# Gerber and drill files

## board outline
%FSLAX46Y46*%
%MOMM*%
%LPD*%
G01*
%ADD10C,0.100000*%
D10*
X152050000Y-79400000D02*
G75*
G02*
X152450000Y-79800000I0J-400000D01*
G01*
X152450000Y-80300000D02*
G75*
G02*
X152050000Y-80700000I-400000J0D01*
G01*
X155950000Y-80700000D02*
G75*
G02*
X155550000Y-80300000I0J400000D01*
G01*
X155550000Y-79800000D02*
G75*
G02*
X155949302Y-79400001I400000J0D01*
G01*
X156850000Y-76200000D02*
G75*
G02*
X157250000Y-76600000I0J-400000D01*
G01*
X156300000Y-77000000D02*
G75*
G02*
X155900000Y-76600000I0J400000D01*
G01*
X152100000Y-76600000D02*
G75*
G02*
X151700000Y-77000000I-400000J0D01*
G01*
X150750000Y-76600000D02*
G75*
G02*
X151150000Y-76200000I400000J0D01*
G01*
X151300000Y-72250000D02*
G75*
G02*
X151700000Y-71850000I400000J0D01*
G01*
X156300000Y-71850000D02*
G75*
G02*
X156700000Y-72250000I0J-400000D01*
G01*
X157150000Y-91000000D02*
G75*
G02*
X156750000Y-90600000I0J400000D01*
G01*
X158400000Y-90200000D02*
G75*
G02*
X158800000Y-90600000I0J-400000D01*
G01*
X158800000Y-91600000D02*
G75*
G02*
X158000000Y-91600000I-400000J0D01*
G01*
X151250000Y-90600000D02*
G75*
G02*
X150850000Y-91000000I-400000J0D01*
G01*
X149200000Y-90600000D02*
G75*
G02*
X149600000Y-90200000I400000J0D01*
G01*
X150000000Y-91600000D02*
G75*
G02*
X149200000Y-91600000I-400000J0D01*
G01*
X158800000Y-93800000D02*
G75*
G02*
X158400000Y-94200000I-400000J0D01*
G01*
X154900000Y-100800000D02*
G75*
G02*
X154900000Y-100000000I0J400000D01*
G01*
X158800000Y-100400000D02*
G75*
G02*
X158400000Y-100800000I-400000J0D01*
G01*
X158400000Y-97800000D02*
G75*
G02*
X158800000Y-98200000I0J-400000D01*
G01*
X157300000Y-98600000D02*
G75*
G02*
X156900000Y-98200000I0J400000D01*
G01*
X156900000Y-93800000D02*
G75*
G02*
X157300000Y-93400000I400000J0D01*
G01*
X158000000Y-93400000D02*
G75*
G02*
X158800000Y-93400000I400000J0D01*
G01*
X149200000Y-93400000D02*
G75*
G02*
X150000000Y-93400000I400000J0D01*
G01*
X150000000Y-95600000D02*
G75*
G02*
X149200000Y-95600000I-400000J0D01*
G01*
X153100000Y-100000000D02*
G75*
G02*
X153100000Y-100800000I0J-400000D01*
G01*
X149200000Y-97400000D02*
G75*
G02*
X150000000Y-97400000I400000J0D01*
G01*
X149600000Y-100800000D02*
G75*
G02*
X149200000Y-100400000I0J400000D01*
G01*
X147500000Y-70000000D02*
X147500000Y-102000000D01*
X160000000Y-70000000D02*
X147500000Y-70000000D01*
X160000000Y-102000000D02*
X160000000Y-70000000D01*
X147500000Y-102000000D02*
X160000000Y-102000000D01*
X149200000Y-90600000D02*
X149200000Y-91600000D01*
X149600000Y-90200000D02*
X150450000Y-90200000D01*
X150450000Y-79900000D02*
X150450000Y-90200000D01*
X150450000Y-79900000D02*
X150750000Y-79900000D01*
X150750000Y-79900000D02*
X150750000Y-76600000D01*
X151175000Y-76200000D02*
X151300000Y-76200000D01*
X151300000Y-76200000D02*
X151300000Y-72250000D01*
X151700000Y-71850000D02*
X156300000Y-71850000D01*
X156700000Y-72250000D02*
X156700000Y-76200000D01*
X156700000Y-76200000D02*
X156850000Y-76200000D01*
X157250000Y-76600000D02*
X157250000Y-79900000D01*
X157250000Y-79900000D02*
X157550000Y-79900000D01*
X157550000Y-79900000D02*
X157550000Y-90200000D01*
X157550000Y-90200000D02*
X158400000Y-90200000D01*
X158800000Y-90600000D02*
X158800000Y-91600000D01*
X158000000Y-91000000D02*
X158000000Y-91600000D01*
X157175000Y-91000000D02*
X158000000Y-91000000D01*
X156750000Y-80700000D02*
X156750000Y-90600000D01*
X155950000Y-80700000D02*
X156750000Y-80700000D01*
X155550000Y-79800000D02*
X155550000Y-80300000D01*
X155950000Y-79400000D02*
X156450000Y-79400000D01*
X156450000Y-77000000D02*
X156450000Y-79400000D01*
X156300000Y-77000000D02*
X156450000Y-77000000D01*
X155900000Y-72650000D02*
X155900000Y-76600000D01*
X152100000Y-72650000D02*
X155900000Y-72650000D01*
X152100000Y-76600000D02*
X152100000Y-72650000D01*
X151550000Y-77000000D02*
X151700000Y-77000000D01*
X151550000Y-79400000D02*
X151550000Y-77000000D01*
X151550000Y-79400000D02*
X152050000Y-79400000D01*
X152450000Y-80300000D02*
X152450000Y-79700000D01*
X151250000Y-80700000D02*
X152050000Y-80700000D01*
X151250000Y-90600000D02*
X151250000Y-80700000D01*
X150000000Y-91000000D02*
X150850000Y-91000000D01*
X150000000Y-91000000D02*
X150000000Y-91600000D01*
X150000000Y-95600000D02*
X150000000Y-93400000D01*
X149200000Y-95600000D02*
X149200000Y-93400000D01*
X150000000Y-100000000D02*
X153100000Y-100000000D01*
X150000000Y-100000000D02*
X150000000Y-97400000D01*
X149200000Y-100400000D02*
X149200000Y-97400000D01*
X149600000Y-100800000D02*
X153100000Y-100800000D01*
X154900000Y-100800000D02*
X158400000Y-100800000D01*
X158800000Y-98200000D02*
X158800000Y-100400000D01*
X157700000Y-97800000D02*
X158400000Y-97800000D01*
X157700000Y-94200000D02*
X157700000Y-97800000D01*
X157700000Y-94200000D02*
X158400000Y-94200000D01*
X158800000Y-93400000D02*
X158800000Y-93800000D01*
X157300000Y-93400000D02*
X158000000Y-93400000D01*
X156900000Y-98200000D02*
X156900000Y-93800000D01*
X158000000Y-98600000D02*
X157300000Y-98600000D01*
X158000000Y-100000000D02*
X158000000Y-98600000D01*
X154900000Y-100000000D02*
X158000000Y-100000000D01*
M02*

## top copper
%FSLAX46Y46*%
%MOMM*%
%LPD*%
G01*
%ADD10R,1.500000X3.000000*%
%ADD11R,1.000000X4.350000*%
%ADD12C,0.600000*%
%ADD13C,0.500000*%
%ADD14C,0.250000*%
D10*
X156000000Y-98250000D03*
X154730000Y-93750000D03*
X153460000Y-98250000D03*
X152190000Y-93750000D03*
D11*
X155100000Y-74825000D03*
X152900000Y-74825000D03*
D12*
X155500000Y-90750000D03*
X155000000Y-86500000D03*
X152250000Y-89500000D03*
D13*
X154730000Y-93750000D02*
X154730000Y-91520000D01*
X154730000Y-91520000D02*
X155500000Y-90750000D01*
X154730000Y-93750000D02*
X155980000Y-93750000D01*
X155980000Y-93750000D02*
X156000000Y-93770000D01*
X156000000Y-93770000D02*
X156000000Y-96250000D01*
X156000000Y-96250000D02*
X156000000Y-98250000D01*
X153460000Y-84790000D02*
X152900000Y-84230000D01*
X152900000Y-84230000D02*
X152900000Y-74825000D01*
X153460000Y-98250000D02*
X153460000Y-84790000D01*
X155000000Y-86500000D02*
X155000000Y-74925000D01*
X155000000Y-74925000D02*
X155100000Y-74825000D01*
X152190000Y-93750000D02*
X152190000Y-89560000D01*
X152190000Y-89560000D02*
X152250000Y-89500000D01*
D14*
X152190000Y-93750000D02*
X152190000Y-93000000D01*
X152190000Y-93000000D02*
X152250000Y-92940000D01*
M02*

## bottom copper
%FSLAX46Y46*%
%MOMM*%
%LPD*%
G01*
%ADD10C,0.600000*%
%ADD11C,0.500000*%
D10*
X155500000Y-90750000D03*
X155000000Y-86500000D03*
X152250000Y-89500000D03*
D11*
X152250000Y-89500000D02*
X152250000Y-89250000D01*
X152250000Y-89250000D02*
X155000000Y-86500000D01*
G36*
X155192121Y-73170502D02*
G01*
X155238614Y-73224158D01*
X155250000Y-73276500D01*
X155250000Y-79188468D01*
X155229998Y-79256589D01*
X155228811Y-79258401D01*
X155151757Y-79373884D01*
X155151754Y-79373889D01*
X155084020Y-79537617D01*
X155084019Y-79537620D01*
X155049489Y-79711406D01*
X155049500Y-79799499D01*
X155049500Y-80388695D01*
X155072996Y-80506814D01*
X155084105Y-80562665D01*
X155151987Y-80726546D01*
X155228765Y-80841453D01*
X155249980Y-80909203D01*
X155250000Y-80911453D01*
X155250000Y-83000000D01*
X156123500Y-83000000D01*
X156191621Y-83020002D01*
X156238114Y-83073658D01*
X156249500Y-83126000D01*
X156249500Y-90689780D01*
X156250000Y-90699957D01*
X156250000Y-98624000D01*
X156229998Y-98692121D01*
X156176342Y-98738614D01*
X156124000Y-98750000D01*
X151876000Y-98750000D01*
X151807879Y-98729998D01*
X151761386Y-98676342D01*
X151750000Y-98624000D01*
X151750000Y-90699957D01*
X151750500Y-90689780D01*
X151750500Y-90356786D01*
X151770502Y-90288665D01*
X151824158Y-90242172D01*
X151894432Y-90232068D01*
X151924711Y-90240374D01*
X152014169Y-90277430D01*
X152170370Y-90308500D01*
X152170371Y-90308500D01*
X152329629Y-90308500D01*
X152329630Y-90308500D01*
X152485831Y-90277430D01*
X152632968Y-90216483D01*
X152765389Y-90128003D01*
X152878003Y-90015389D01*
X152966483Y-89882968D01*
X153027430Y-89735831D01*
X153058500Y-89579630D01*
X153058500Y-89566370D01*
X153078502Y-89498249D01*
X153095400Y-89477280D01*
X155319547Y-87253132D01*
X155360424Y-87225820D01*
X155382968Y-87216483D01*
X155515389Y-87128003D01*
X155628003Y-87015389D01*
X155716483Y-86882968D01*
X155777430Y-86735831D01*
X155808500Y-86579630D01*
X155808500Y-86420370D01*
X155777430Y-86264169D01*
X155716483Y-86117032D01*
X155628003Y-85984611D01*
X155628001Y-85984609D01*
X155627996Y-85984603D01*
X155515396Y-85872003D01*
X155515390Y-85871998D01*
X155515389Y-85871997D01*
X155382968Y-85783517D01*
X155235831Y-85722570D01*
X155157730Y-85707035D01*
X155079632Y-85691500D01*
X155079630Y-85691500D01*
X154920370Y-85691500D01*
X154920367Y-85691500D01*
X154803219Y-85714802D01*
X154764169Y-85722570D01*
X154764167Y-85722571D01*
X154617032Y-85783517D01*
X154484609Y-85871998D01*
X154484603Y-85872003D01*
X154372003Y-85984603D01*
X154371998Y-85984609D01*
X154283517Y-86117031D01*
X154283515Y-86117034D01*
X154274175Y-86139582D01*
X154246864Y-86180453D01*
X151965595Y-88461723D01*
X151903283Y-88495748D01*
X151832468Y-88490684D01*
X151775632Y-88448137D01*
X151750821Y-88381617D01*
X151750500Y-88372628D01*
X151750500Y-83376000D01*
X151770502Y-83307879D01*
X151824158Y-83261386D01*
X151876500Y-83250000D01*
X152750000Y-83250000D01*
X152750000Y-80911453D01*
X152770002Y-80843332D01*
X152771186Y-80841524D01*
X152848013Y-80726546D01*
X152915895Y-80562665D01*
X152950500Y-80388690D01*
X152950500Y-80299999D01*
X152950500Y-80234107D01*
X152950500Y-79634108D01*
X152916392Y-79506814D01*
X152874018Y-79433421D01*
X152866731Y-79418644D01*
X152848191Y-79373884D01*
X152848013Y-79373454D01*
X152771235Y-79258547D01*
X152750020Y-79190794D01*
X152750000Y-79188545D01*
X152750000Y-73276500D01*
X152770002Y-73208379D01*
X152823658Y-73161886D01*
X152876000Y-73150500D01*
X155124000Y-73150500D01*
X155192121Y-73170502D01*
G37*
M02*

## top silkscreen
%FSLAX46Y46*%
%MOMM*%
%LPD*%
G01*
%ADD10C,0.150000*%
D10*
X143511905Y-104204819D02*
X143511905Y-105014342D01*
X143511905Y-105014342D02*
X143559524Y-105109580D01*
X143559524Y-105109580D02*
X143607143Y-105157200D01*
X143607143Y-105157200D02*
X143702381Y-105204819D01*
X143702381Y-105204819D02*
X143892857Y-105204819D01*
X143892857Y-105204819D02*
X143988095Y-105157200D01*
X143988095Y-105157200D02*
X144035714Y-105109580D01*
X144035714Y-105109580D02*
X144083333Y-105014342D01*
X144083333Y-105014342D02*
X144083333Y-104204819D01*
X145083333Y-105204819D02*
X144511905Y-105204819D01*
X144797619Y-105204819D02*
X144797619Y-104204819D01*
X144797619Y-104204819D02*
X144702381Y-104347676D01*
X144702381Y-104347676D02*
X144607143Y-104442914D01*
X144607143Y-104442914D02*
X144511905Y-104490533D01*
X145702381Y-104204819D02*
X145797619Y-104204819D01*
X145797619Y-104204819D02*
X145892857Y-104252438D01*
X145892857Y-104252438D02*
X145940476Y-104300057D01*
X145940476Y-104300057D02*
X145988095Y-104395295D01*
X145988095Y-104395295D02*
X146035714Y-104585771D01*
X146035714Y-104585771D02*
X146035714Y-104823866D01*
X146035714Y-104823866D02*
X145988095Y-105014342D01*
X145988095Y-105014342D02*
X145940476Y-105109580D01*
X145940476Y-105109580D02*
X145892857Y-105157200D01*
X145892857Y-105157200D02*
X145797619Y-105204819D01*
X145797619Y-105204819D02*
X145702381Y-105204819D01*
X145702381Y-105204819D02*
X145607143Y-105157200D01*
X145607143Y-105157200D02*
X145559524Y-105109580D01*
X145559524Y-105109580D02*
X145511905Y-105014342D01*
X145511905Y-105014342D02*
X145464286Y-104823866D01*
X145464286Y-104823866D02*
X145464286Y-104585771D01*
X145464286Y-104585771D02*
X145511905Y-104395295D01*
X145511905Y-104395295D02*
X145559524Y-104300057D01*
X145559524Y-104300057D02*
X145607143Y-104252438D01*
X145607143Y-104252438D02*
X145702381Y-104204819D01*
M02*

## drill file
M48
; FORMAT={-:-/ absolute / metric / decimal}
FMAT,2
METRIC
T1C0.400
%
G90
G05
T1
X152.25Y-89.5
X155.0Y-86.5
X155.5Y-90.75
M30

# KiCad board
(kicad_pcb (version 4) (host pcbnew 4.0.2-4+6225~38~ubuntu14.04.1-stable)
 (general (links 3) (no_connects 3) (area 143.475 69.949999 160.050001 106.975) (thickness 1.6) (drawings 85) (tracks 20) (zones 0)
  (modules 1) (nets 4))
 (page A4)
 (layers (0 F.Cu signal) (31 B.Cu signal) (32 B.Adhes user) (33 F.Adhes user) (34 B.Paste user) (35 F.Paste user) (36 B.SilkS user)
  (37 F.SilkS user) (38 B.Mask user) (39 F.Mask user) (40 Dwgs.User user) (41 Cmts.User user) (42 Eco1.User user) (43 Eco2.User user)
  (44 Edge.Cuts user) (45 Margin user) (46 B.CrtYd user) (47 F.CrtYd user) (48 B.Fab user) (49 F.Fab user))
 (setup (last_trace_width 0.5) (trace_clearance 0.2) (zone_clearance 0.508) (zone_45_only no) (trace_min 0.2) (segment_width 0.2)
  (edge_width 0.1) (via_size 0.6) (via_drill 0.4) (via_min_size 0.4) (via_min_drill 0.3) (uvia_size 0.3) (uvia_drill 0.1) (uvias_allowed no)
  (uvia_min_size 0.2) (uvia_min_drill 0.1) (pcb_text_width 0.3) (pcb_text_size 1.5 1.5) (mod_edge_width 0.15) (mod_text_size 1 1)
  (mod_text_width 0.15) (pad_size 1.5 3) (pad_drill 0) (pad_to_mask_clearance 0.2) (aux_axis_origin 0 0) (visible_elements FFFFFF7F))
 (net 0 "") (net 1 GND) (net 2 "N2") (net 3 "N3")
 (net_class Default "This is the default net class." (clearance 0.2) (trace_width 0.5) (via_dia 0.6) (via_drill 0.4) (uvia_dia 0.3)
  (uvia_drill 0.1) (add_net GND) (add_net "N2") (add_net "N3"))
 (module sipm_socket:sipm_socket (layer F.Cu) (at 150 100)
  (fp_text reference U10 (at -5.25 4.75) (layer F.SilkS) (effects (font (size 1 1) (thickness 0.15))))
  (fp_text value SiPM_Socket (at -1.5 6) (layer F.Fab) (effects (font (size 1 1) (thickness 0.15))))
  (pad 1 smd rect (at 6 -1.75) (size 1.5 3) (layers F.Cu F.Paste F.Mask) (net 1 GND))
  (pad 2 smd rect (at 4.73 -6.25) (size 1.5 3) (layers F.Cu F.Paste F.Mask) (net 1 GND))
  (pad 3 smd rect (at 3.46 -1.75) (size 1.5 3) (layers F.Cu F.Paste F.Mask) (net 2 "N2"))
  (pad 4 smd rect (at 2.19 -6.25) (size 1.5 3) (layers F.Cu F.Paste F.Mask) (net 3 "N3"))
  (pad 5 smd rect (at 5.1 -25.175) (size 1 4.35) (layers F.Cu F.Paste F.Mask) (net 3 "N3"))
  (pad 6 smd rect (at 2.9 -25.175) (size 1 4.35) (layers F.Cu F.Paste F.Mask) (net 2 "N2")))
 (gr_arc (start 152.05 79.8) (end 152.05 79.4) (angle 90) (layer Edge.Cuts) (width 0.1))
 (gr_arc (start 152.05 80.3) (end 152.45 80.3) (angle 90) (layer Edge.Cuts) (width 0.1))
 (gr_arc (start 155.95 80.3) (end 155.55 80.3) (angle -90) (layer Edge.Cuts) (width 0.1))
 (gr_arc (start 155.95 79.8) (end 155.55 79.8) (angle 89.9) (layer Edge.Cuts) (width 0.1))
 (gr_arc (start 156.85 76.6) (end 157.25 76.6) (angle -90) (layer Edge.Cuts) (width 0.1))
 (gr_arc (start 156.3 76.6) (end 156.3 77) (angle 90) (layer Edge.Cuts) (width 0.1))
 (gr_arc (start 151.7 76.6) (end 152.1 76.6) (angle 90) (layer Edge.Cuts) (width 0.1))
 (gr_arc (start 151.15 76.6) (end 150.75 76.6) (angle 90) (layer Edge.Cuts) (width 0.1))
 (gr_arc (start 151.7 72.25) (end 151.3 72.25) (angle 90) (layer Edge.Cuts) (width 0.1))
 (gr_arc (start 156.3 72.25) (end 156.7 72.25) (angle -90) (layer Edge.Cuts) (width 0.1))
 (gr_arc (start 157.15 90.6) (end 156.75 90.6) (angle -90) (layer Edge.Cuts) (width 0.1))
 (gr_arc (start 158.4 90.6) (end 158.4 90.2) (angle 90) (layer Edge.Cuts) (width 0.1))
 (gr_arc (start 158.4 91.6) (end 158 91.6) (angle -180) (layer Edge.Cuts) (width 0.1))
 (gr_arc (start 150.85 90.6) (end 150.85 91) (angle -90) (layer Edge.Cuts) (width 0.1))
 (gr_arc (start 149.6 90.6) (end 149.2 90.6) (angle 90) (layer Edge.Cuts) (width 0.1))
 (gr_arc (start 149.6 91.6) (end 149.2 91.6) (angle -180) (layer Edge.Cuts) (width 0.1))
 (gr_arc (start 158.4 93.8) (end 158.8 93.8) (angle 90) (layer Edge.Cuts) (width 0.1))
 (gr_arc (start 154.9 100.4) (end 154.9 100) (angle -180) (layer Edge.Cuts) (width 0.1))
 (gr_arc (start 158.4 100.4) (end 158.4 100.8) (angle -90) (layer Edge.Cuts) (width 0.1))
 (gr_arc (start 158.4 98.2) (end 158.8 98.2) (angle -90) (layer Edge.Cuts) (width 0.1))
 (gr_arc (start 157.3 98.2) (end 156.9 98.2) (angle -90) (layer Edge.Cuts) (width 0.1))
 (gr_arc (start 157.3 93.8) (end 156.9 93.8) (angle 90) (layer Edge.Cuts) (width 0.1))
 (gr_arc (start 158.4 93.4) (end 158 93.4) (angle 180) (layer Edge.Cuts) (width 0.1))
 (gr_arc (start 149.6 93.4) (end 149.2 93.4) (angle 180) (layer Edge.Cuts) (width 0.1))
 (gr_arc (start 149.6 95.6) (end 149.2 95.6) (angle -180) (layer Edge.Cuts) (width 0.1))
 (gr_arc (start 153.1 100.4) (end 153.1 100) (angle 180) (layer Edge.Cuts) (width 0.1))
 (gr_arc (start 149.6 97.4) (end 150 97.4) (angle -180) (layer Edge.Cuts) (width 0.1))
 (gr_arc (start 149.6 100.4) (end 149.2 100.4) (angle -90) (layer Edge.Cuts) (width 0.1))
 (gr_line (start 147.5 70) (end 147.5 102) (layer Edge.Cuts) (width 0.1))
 (gr_line (start 160 70) (end 147.5 70) (layer Edge.Cuts) (width 0.1))
 (gr_line (start 160 102) (end 160 70) (layer Edge.Cuts) (width 0.1))
 (gr_line (start 147.5 102) (end 160 102) (layer Edge.Cuts) (width 0.1))
 (gr_line (start 149.2 90.6) (end 149.2 91.6) (layer Edge.Cuts) (width 0.1))
 (gr_line (start 149.6 90.2) (end 150.45 90.2) (layer Edge.Cuts) (width 0.1))
 (gr_line (start 150.45 79.9) (end 150.45 90.2) (layer Edge.Cuts) (width 0.1))
 (gr_line (start 150.45 79.9) (end 150.75 79.9) (layer Edge.Cuts) (width 0.1))
 (gr_line (start 150.75 79.9) (end 150.75 76.6) (layer Edge.Cuts) (width 0.1))
 (gr_line (start 151.175 76.2) (end 151.3 76.2) (layer Edge.Cuts) (width 0.1))
 (gr_line (start 151.3 76.2) (end 151.3 72.25) (layer Edge.Cuts) (width 0.1))
 (gr_line (start 151.7 71.85) (end 156.3 71.85) (layer Edge.Cuts) (width 0.1))
 (gr_line (start 156.7 72.25) (end 156.7 76.2) (layer Edge.Cuts) (width 0.1))
 (gr_line (start 156.7 76.2) (end 156.85 76.2) (layer Edge.Cuts) (width 0.1))
 (gr_line (start 157.25 76.6) (end 157.25 79.9) (layer Edge.Cuts) (width 0.1))
 (gr_line (start 157.25 79.9) (end 157.55 79.9) (layer Edge.Cuts) (width 0.1))
 (gr_line (start 157.55 79.9) (end 157.55 90.2) (layer Edge.Cuts) (width 0.1))
 (gr_line (start 157.55 90.2) (end 158.4 90.2) (layer Edge.Cuts) (width 0.1))
 (gr_line (start 158.8 90.6) (end 158.8 91.6) (layer Edge.Cuts) (width 0.1))
 (gr_line (start 158 91) (end 158 91.6) (layer Edge.Cuts) (width 0.1))
 (gr_line (start 157.175 91) (end 158 91) (layer Edge.Cuts) (width 0.1))
 (gr_line (start 156.75 80.7) (end 156.75 90.6) (layer Edge.Cuts) (width 0.1))
 (gr_line (start 155.95 80.7) (end 156.75 80.7) (layer Edge.Cuts) (width 0.1))
 (gr_line (start 155.55 79.8) (end 155.55 80.3) (layer Edge.Cuts) (width 0.1))
 (gr_line (start 155.95 79.4) (end 156.45 79.4) (layer Edge.Cuts) (width 0.1))
 (gr_line (start 156.45 77) (end 156.45 79.4) (layer Edge.Cuts) (width 0.1))
 (gr_line (start 156.3 77) (end 156.45 77) (layer Edge.Cuts) (width 0.1))
 (gr_line (start 155.9 72.65) (end 155.9 76.6) (layer Edge.Cuts) (width 0.1))
 (gr_line (start 152.1 72.65) (end 155.9 72.65) (layer Edge.Cuts) (width 0.1))
 (gr_line (start 152.1 76.6) (end 152.1 72.65) (layer Edge.Cuts) (width 0.1))
 (gr_line (start 151.55 77) (end 151.7 77) (layer Edge.Cuts) (width 0.1))
 (gr_line (start 151.55 79.4) (end 151.55 77) (layer Edge.Cuts) (width 0.1))
 (gr_line (start 151.55 79.4) (end 152.05 79.4) (layer Edge.Cuts) (width 0.1))
 (gr_line (start 152.45 80.3) (end 152.45 79.7) (layer Edge.Cuts) (width 0.1))
 (gr_line (start 151.25 80.7) (end 152.05 80.7) (layer Edge.Cuts) (width 0.1))
 (gr_line (start 151.25 90.6) (end 151.25 80.7) (layer Edge.Cuts) (width 0.1))
 (gr_line (start 150 91) (end 150.85 91) (layer Edge.Cuts) (width 0.1))
 (gr_line (start 150 91) (end 150 91.6) (layer Edge.Cuts) (width 0.1))
 (gr_line (start 150 95.6) (end 150 93.4) (layer Edge.Cuts) (width 0.1))
 (gr_line (start 149.2 95.6) (end 149.2 93.4) (layer Edge.Cuts) (width 0.1))
 (gr_line (start 150 100) (end 153.1 100) (layer Edge.Cuts) (width 0.1))
 (gr_line (start 150 100) (end 150 97.4) (layer Edge.Cuts) (width 0.1))
 (gr_line (start 149.2 100.4) (end 149.2 97.4) (layer Edge.Cuts) (width 0.1))
 (gr_line (start 149.6 100.8) (end 153.1 100.8) (layer Edge.Cuts) (width 0.1))
 (gr_line (start 154.9 100.8) (end 158.4 100.8) (layer Edge.Cuts) (width 0.1))
 (gr_line (start 158.8 98.2) (end 158.8 100.4) (layer Edge.Cuts) (width 0.1))
 (gr_line (start 157.7 97.8) (end 158.4 97.8) (layer Edge.Cuts) (width 0.1))
 (gr_line (start 157.7 94.2) (end 157.7 97.8) (layer Edge.Cuts) (width 0.1))
 (gr_line (start 157.7 94.2) (end 158.4 94.2) (layer Edge.Cuts) (width 0.1))
 (gr_line (start 158.8 93.4) (end 158.8 93.8) (layer Edge.Cuts) (width 0.1))
 (gr_line (start 157.3 93.4) (end 158 93.4) (layer Edge.Cuts) (width 0.1))
 (gr_line (start 156.9 98.2) (end 156.9 93.8) (layer Edge.Cuts) (width 0.1))
 (gr_line (start 158 98.6) (end 157.3 98.6) (layer Edge.Cuts) (width 0.1))
 (gr_line (start 158 100) (end 158 98.6) (layer Edge.Cuts) (width 0.1))
 (gr_line (start 154.9 100) (end 158 100) (layer Edge.Cuts) (width 0.1))
 (segment (start 154.73 93.75) (end 154.73 91.52) (width 0.5) (layer F.Cu) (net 1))
 (segment (start 154.73 91.52) (end 155.5 90.75) (width 0.5) (layer F.Cu) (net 1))
 (via (at 155.5 90.75) (size 0.6) (drill 0.4) (layers F.Cu B.Cu) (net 1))
 (segment (start 154.73 93.75) (end 155.98 93.75) (width 0.5) (layer F.Cu) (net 1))
 (segment (start 155.98 93.75) (end 156 93.77) (width 0.5) (layer F.Cu) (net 1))
 (segment (start 156 93.77) (end 156 96.25) (width 0.5) (layer F.Cu) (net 1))
 (segment (start 156 96.25) (end 156 98.25) (width 0.5) (layer F.Cu) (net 1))
 (segment (start 153.46 84.79) (end 152.9 84.23) (width 0.5) (layer F.Cu) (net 2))
 (segment (start 152.9 84.23) (end 152.9 74.825) (width 0.5) (layer F.Cu) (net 2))
 (segment (start 153.46 98.25) (end 153.46 84.79) (width 0.5) (layer F.Cu) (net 2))
 (segment (start 155 86.5) (end 155 74.925) (width 0.5) (layer F.Cu) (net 3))
 (segment (start 155 74.925) (end 155.1 74.825) (width 0.5) (layer F.Cu) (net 3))
 (segment (start 152.25 89.5) (end 152.25 89.25) (width 0.5) (layer B.Cu) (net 3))
 (segment (start 152.25 89.25) (end 155 86.5) (width 0.5) (layer B.Cu) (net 3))
 (via (at 155 86.5) (size 0.6) (drill 0.4) (layers F.Cu B.Cu) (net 3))
 (segment (start 152.19 93.75) (end 152.19 89.56) (width 0.5) (layer F.Cu) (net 3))
 (segment (start 152.19 89.56) (end 152.25 89.5) (width 0.5) (layer F.Cu) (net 3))
 (via (at 152.25 89.5) (size 0.6) (drill 0.4) (layers F.Cu B.Cu) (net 3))
 (segment (start 152.19 93.75) (end 152.19 93) (width 0.25) (layer F.Cu) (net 3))
 (segment (start 152.19 93) (end 152.25 92.94) (width 0.25) (layer F.Cu) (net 3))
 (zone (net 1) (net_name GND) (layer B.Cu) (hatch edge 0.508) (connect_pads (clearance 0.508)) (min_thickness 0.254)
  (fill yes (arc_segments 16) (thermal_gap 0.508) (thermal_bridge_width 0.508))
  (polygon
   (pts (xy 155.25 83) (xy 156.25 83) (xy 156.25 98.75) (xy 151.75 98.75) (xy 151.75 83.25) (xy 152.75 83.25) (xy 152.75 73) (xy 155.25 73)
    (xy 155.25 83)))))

